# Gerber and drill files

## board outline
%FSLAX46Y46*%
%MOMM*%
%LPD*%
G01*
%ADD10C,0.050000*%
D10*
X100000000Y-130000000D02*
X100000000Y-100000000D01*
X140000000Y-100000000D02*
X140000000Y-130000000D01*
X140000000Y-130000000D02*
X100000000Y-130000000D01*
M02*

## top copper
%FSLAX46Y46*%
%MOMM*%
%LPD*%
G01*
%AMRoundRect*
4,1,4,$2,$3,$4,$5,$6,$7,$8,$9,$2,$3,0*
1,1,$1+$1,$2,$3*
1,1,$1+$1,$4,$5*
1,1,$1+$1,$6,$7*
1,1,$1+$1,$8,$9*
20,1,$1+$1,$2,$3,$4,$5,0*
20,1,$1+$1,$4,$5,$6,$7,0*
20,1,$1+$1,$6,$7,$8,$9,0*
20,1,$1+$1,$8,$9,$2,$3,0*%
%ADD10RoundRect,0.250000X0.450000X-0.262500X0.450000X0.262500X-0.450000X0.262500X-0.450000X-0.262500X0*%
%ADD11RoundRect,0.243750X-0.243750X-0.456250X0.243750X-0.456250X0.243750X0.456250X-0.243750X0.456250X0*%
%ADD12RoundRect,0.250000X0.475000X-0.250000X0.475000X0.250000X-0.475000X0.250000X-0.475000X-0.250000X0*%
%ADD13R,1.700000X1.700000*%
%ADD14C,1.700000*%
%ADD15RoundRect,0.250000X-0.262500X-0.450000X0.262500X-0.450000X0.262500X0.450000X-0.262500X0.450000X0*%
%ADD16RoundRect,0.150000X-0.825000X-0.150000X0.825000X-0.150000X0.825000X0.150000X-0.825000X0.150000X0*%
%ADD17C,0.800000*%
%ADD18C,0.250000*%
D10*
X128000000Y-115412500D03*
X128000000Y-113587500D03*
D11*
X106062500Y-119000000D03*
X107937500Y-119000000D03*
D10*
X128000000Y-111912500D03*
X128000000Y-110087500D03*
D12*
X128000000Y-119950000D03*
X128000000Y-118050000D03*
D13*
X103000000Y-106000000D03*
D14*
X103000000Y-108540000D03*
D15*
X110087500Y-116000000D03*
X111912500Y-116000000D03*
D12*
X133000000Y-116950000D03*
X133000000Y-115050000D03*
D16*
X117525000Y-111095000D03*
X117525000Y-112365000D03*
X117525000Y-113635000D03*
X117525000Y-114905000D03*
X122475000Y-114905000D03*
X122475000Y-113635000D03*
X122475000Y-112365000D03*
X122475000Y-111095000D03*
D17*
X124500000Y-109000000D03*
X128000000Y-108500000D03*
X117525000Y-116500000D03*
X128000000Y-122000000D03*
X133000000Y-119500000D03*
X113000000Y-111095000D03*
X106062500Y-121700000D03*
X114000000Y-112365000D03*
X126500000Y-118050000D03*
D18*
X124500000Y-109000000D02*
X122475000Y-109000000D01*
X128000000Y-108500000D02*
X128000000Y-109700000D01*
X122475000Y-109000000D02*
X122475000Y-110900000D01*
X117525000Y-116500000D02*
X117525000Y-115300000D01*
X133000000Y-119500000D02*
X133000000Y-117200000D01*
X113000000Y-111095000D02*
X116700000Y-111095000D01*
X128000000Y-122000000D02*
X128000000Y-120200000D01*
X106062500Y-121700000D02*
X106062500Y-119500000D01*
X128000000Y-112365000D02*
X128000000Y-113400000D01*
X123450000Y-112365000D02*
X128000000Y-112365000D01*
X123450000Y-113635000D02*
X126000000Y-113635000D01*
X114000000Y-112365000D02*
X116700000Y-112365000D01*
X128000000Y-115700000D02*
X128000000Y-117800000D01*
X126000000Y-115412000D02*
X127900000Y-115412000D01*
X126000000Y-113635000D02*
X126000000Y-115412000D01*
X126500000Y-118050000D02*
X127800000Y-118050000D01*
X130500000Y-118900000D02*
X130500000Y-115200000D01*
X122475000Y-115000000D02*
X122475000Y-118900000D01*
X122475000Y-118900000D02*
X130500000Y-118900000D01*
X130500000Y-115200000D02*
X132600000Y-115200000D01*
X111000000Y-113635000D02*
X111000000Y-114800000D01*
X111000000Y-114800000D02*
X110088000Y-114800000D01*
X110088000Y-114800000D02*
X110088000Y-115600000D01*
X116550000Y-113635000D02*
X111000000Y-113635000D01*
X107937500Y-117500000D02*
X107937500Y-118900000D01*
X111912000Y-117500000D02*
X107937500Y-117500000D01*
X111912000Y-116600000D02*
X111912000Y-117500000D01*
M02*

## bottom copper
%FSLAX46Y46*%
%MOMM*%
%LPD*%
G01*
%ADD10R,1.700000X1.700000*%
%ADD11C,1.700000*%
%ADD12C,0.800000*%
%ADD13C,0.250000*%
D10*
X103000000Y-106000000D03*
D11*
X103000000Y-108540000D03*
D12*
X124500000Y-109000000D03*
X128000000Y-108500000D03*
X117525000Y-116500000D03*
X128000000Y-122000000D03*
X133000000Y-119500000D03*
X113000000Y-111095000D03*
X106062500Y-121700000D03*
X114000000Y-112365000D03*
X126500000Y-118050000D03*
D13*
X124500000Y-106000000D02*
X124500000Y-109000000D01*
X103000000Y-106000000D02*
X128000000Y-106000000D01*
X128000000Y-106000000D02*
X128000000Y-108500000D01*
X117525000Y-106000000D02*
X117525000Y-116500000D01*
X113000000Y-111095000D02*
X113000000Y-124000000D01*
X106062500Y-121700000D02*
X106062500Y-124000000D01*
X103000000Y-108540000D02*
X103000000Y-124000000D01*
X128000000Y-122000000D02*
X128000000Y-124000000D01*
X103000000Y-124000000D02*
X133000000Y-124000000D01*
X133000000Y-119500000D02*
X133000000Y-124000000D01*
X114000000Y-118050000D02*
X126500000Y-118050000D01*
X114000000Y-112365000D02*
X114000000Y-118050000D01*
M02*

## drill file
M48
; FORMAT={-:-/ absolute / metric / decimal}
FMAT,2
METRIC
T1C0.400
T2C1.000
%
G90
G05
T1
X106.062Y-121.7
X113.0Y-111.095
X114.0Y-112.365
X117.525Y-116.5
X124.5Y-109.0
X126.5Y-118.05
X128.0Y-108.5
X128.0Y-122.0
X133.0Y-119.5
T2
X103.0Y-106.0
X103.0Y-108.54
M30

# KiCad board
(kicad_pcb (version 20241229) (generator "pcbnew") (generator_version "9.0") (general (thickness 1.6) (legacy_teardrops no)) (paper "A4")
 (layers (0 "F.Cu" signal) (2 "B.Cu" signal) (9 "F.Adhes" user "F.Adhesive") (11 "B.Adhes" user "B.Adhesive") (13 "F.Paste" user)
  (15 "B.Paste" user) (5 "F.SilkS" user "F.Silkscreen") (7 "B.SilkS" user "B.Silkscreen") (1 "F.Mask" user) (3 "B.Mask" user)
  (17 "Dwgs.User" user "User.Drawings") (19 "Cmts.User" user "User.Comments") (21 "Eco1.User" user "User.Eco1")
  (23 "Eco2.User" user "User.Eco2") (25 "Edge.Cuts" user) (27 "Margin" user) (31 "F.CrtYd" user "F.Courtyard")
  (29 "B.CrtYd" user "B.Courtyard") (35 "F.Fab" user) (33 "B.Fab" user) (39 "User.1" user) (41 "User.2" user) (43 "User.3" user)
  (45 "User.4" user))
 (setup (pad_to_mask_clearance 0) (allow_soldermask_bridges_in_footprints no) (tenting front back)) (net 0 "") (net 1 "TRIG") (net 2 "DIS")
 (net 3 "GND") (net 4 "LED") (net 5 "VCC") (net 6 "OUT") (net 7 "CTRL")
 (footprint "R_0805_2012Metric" (layer "F.Cu") (at 128 114.5 90)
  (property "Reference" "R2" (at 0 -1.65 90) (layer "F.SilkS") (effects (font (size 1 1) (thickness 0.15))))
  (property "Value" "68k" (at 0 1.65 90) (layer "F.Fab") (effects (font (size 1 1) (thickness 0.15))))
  (pad "1" smd roundrect (at -0.9125 0 90) (size 1.025 1.4) (layers "F.Cu" "F.Mask" "F.Paste") (roundrect_rratio 0.243902) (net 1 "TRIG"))
  (pad "2" smd roundrect (at 0.9125 0 90) (size 1.025 1.4) (layers "F.Cu" "F.Mask" "F.Paste") (roundrect_rratio 0.243902) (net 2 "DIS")))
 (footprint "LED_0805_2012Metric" (layer "F.Cu") (at 107 119)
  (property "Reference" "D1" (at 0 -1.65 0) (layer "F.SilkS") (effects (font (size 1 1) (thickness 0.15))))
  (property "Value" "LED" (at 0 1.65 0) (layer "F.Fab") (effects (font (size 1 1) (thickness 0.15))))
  (pad "1" smd roundrect (at -0.9375 0) (size 0.975 1.4) (layers "F.Cu" "F.Mask" "F.Paste") (roundrect_rratio 0.25) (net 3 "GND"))
  (pad "2" smd roundrect (at 0.9375 0) (size 0.975 1.4) (layers "F.Cu" "F.Mask" "F.Paste") (roundrect_rratio 0.25) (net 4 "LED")))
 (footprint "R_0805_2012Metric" (layer "F.Cu") (at 128 111 90)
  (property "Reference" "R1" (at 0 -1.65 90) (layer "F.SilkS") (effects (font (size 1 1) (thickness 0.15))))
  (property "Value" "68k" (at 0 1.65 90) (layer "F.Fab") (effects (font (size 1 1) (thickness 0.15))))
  (pad "1" smd roundrect (at -0.9125 0 90) (size 1.025 1.4) (layers "F.Cu" "F.Mask" "F.Paste") (roundrect_rratio 0.243902) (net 2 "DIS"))
  (pad "2" smd roundrect (at 0.9125 0 90) (size 1.025 1.4) (layers "F.Cu" "F.Mask" "F.Paste") (roundrect_rratio 0.243902) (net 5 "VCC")))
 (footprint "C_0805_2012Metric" (layer "F.Cu") (at 128 119 90)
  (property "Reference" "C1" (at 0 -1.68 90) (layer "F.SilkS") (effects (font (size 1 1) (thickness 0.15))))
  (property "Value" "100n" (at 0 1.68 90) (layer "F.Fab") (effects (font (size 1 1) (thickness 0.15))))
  (pad "1" smd roundrect (at -0.95 0 90) (size 1 1.45) (layers "F.Cu" "F.Mask" "F.Paste") (roundrect_rratio 0.25) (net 3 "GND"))
  (pad "2" smd roundrect (at 0.95 0 90) (size 1 1.45) (layers "F.Cu" "F.Mask" "F.Paste") (roundrect_rratio 0.25) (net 1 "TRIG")))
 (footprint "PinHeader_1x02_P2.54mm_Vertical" (layer "F.Cu") (at 103 106)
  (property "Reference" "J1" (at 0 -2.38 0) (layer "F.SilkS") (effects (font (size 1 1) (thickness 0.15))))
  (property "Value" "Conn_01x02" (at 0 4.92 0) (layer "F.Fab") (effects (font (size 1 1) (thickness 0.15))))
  (pad "1" thru_hole rect (at 0 0) (size 1.7 1.7) (drill 1) (layers "*.Cu" "*.Mask") (remove_unused_layers no) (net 5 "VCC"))
  (pad "2" thru_hole circle (at 0 2.54) (size 1.7 1.7) (drill 1) (layers "*.Cu" "*.Mask") (remove_unused_layers no) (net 3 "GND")))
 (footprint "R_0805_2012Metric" (layer "F.Cu") (at 111 116)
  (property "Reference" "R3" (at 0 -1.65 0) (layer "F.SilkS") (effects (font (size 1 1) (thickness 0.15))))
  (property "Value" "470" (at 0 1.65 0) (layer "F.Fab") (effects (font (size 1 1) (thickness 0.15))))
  (pad "1" smd roundrect (at -0.9125 0) (size 1.025 1.4) (layers "F.Cu" "F.Mask" "F.Paste") (roundrect_rratio 0.243902) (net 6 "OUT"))
  (pad "2" smd roundrect (at 0.9125 0) (size 1.025 1.4) (layers "F.Cu" "F.Mask" "F.Paste") (roundrect_rratio 0.243902) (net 4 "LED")))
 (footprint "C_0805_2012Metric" (layer "F.Cu") (at 133 116 90)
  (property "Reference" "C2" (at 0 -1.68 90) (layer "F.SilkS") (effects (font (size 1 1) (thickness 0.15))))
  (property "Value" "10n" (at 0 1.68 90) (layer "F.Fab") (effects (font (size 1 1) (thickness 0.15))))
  (pad "1" smd roundrect (at -0.95 0 90) (size 1 1.45) (layers "F.Cu" "F.Mask" "F.Paste") (roundrect_rratio 0.25) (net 3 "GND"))
  (pad "2" smd roundrect (at 0.95 0 90) (size 1 1.45) (layers "F.Cu" "F.Mask" "F.Paste") (roundrect_rratio 0.25) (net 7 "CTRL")))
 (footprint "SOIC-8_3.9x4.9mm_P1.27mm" (layer "F.Cu") (at 120 113)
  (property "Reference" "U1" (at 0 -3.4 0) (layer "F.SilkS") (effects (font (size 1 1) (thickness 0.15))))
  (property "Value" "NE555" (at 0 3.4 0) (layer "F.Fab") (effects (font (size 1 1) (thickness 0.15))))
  (pad "1" smd roundrect (at -2.475 -1.905) (size 1.95 0.6) (layers "F.Cu" "F.Mask" "F.Paste") (roundrect_rratio 0.25) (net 3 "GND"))
  (pad "2" smd roundrect (at -2.475 -0.635) (size 1.95 0.6) (layers "F.Cu" "F.Mask" "F.Paste") (roundrect_rratio 0.25) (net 1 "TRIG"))
  (pad "3" smd roundrect (at -2.475 0.635) (size 1.95 0.6) (layers "F.Cu" "F.Mask" "F.Paste") (roundrect_rratio 0.25) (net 6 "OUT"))
  (pad "4" smd roundrect (at -2.475 1.905) (size 1.95 0.6) (layers "F.Cu" "F.Mask" "F.Paste") (roundrect_rratio 0.25) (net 5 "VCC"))
  (pad "5" smd roundrect (at 2.475 1.905) (size 1.95 0.6) (layers "F.Cu" "F.Mask" "F.Paste") (roundrect_rratio 0.25) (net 7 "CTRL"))
  (pad "6" smd roundrect (at 2.475 0.635) (size 1.95 0.6) (layers "F.Cu" "F.Mask" "F.Paste") (roundrect_rratio 0.25) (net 1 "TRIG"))
  (pad "7" smd roundrect (at 2.475 -0.635) (size 1.95 0.6) (layers "F.Cu" "F.Mask" "F.Paste") (roundrect_rratio 0.25) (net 2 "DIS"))
  (pad "8" smd roundrect (at 2.475 -1.905) (size 1.95 0.6) (layers "F.Cu" "F.Mask" "F.Paste") (roundrect_rratio 0.25) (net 5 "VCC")))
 (gr_line (start 100 130) (end 100 100) (stroke (width 0.05) (type default)) (layer "Edge.Cuts"))
 (gr_line (start 140 100) (end 140 130) (stroke (width 0.05) (type default)) (layer "Edge.Cuts"))
 (gr_line (start 140 130) (end 100 130) (stroke (width 0.05) (type default)) (layer "Edge.Cuts"))
 (segment (start 124.5 109) (end 122.475 109) (width 0.25) (layer "F.Cu") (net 5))
 (segment (start 128 108.5) (end 128 109.7) (width 0.25) (layer "F.Cu") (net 5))
 (segment (start 122.475 109) (end 122.475 110.9) (width 0.25) (layer "F.Cu") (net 5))
 (segment (start 117.525 116.5) (end 117.525 115.3) (width 0.25) (layer "F.Cu") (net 5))
 (via (at 124.5 109) (size 0.8) (drill 0.4) (layers "F.Cu" "B.Cu") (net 5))
 (via (at 128 108.5) (size 0.8) (drill 0.4) (layers "F.Cu" "B.Cu") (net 5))
 (via (at 117.525 116.5) (size 0.8) (drill 0.4) (layers "F.Cu" "B.Cu") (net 5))
 (segment (start 124.5 106) (end 124.5 109) (width 0.25) (layer "B.Cu") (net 5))
 (segment (start 103 106) (end 128 106) (width 0.25) (layer "B.Cu") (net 5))
 (segment (start 128 106) (end 128 108.5) (width 0.25) (layer "B.Cu") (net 5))
 (segment (start 117.525 106) (end 117.525 116.5) (width 0.25) (layer "B.Cu") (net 5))
 (segment (start 133 119.5) (end 133 117.2) (width 0.25) (layer "F.Cu") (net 3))
 (segment (start 113 111.095) (end 116.7 111.095) (width 0.25) (layer "F.Cu") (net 3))
 (segment (start 128 122) (end 128 120.2) (width 0.25) (layer "F.Cu") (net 3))
 (segment (start 106.0625 121.7) (end 106.0625 119.5) (width 0.25) (layer "F.Cu") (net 3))
 (via (at 128 122) (size 0.8) (drill 0.4) (layers "F.Cu" "B.Cu") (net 3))
 (via (at 133 119.5) (size 0.8) (drill 0.4) (layers "F.Cu" "B.Cu") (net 3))
 (via (at 113 111.095) (size 0.8) (drill 0.4) (layers "F.Cu" "B.Cu") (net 3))
 (via (at 106.0625 121.7) (size 0.8) (drill 0.4) (layers "F.Cu" "B.Cu") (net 3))
 (segment (start 113 111.095) (end 113 124) (width 0.25) (layer "B.Cu") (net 3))
 (segment (start 106.0625 121.7) (end 106.0625 124) (width 0.25) (layer "B.Cu") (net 3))
 (segment (start 103 108.54) (end 103 124) (width 0.25) (layer "B.Cu") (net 3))
 (segment (start 128 122) (end 128 124) (width 0.25) (layer "B.Cu") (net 3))
 (segment (start 103 124) (end 133 124) (width 0.25) (layer "B.Cu") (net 3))
 (segment (start 133 119.5) (end 133 124) (width 0.25) (layer "B.Cu") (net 3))
 (segment (start 128 112.365) (end 128 113.4) (width 0.25) (layer "F.Cu") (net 2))
 (segment (start 123.45 112.365) (end 128 112.365) (width 0.25) (layer "F.Cu") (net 2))
 (segment (start 123.45 113.635) (end 126 113.635) (width 0.25) (layer "F.Cu") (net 1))
 (segment (start 114 112.365) (end 116.7 112.365) (width 0.25) (layer "F.Cu") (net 1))
 (segment (start 128 115.7) (end 128 117.8) (width 0.25) (layer "F.Cu") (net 1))
 (segment (start 126 115.412) (end 127.9 115.412) (width 0.25) (layer "F.Cu") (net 1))
 (segment (start 126 113.635) (end 126 115.412) (width 0.25) (layer "F.Cu") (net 1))
 (segment (start 126.5 118.05) (end 127.8 118.05) (width 0.25) (layer "F.Cu") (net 1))
 (via (at 114 112.365) (size 0.8) (drill 0.4) (layers "F.Cu" "B.Cu") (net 1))
 (via (at 126.5 118.05) (size 0.8) (drill 0.4) (layers "F.Cu" "B.Cu") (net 1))
 (segment (start 114 118.05) (end 126.5 118.05) (width 0.25) (layer "B.Cu") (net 1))
 (segment (start 114 112.365) (end 114 118.05) (width 0.25) (layer "B.Cu") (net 1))
 (segment (start 130.5 118.9) (end 130.5 115.2) (width 0.25) (layer "F.Cu") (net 7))
 (segment (start 122.475 115) (end 122.475 118.9) (width 0.25) (layer "F.Cu") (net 7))
 (segment (start 122.475 118.9) (end 130.5 118.9) (width 0.25) (layer "F.Cu") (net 7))
 (segment (start 130.5 115.2) (end 132.6 115.2) (width 0.25) (layer "F.Cu") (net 7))
 (segment (start 111 113.635) (end 111 114.8) (width 0.25) (layer "F.Cu") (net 6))
 (segment (start 111 114.8) (end 110.088 114.8) (width 0.25) (layer "F.Cu") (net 6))
 (segment (start 110.088 114.8) (end 110.088 115.6) (width 0.25) (layer "F.Cu") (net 6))
 (segment (start 116.55 113.635) (end 111 113.635) (width 0.25) (layer "F.Cu") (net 6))
 (segment (start 107.9375 117.5) (end 107.9375 118.9) (width 0.25) (layer "F.Cu") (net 4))
 (segment (start 111.912 117.5) (end 107.9375 117.5) (width 0.25) (layer "F.Cu") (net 4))
 (segment (start 111.912 116.6) (end 111.912 117.5) (width 0.25) (layer "F.Cu") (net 4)))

